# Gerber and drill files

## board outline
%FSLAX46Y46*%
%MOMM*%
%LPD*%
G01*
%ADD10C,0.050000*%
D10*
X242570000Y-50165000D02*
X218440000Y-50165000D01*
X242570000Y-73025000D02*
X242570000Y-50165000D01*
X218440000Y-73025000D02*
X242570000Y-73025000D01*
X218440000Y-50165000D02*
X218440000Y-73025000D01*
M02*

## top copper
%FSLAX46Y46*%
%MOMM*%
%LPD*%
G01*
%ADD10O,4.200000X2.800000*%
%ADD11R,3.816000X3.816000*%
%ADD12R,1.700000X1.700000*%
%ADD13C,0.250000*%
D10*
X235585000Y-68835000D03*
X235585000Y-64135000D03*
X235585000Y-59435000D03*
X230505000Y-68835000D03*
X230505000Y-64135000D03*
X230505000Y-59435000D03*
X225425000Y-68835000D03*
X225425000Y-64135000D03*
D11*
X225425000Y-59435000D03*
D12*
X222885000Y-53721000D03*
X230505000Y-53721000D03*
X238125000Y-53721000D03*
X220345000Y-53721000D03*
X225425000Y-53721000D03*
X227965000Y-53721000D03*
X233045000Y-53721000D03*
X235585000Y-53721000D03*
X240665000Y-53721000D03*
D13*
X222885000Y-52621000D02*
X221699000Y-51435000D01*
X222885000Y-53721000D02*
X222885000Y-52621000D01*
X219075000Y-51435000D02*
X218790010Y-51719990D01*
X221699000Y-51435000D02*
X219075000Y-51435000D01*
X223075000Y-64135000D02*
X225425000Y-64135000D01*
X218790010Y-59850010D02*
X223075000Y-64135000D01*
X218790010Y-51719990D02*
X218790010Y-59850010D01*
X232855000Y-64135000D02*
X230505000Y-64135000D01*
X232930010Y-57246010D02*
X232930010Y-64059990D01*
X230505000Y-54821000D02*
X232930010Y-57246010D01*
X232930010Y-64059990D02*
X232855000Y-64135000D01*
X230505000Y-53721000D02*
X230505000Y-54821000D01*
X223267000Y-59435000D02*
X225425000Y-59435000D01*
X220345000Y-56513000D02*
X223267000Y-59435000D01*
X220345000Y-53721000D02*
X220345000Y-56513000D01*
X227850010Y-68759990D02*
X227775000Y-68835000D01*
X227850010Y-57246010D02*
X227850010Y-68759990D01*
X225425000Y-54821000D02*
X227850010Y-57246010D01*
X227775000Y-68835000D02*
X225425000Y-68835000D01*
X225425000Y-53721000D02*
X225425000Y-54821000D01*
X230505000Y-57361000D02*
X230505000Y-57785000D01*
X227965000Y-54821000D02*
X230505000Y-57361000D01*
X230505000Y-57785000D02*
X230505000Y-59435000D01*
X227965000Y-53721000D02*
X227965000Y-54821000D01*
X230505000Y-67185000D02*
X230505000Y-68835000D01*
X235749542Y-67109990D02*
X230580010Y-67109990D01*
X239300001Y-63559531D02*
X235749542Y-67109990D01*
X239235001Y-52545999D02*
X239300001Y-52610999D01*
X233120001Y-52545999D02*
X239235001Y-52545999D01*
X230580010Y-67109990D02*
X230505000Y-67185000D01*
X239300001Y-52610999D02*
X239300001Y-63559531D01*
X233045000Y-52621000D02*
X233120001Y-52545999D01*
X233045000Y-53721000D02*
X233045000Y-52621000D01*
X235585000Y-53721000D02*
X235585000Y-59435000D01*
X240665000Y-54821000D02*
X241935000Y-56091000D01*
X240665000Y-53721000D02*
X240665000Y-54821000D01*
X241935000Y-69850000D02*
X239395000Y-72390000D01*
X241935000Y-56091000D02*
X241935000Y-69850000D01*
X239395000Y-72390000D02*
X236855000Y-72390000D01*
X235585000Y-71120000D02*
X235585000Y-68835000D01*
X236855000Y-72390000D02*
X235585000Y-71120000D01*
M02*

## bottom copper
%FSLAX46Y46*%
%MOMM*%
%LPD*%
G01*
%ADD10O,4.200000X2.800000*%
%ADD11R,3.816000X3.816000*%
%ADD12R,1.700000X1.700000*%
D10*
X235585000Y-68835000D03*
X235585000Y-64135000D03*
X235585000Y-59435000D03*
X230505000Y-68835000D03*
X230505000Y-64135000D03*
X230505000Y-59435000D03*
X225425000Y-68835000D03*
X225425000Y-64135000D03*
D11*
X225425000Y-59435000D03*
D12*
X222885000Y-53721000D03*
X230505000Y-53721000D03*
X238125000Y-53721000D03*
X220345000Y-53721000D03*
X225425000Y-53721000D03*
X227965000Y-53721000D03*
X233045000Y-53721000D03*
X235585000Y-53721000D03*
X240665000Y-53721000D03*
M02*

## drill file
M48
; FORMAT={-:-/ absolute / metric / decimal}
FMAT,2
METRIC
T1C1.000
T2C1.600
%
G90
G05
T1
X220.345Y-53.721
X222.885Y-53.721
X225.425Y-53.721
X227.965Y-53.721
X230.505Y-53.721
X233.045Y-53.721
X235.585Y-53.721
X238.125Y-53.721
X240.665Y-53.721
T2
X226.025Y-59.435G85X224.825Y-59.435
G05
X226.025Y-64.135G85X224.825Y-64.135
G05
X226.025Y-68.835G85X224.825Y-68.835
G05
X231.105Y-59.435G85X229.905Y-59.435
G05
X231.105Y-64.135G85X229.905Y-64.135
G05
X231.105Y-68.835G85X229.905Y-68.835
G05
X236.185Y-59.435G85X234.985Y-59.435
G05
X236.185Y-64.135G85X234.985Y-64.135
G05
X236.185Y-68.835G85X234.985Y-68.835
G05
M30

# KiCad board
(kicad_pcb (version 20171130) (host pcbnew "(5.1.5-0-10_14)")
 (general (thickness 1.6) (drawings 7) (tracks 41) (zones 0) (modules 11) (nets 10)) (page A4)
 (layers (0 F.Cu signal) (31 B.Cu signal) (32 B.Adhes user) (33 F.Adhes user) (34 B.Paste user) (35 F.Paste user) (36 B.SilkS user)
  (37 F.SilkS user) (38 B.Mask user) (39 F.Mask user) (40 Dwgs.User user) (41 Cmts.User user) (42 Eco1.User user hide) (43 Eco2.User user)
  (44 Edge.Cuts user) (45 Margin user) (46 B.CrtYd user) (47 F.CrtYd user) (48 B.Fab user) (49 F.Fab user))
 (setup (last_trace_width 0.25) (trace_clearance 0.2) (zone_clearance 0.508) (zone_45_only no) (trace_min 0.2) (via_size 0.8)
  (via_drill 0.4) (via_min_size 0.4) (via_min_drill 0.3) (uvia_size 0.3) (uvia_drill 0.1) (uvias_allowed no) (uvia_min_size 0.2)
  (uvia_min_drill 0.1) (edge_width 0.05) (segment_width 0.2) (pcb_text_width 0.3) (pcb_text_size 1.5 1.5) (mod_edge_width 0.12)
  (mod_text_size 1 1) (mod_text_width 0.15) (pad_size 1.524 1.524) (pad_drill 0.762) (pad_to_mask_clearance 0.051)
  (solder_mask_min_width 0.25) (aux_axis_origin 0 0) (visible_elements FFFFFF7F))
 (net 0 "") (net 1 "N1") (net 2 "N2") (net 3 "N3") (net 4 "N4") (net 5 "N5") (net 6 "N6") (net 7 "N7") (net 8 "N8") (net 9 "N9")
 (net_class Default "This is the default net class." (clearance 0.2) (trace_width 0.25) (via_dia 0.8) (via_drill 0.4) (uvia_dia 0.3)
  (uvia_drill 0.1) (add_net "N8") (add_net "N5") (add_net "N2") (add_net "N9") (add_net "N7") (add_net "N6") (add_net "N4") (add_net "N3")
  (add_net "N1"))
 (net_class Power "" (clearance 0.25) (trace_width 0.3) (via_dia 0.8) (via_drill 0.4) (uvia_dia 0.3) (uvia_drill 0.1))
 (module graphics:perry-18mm (layer F.Cu) (at 229.87 62.865)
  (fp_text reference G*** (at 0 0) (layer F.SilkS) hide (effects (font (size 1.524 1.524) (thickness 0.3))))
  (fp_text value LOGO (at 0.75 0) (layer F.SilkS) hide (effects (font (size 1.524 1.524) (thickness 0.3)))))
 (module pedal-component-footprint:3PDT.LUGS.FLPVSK (layer F.Cu) (at 230.505 64.135)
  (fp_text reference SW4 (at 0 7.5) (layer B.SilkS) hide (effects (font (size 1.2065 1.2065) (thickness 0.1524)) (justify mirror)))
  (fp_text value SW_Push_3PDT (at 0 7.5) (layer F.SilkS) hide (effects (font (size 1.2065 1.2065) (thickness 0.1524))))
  (pad 9 thru_hole oval (at 5.08 4.7 180) (size 4.2 2.8) (drill oval 2.8 1.6) (layers *.Cu *.Mask) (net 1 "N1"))
  (pad 8 thru_hole oval (at 5.08 0 180) (size 4.2 2.8) (drill oval 2.8 1.6) (layers *.Cu *.Mask) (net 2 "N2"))
  (pad 7 thru_hole oval (at 5.08 -4.7 180) (size 4.2 2.8) (drill oval 2.8 1.6) (layers *.Cu *.Mask) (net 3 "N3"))
  (pad 6 thru_hole oval (at 0 4.7 180) (size 4.2 2.8) (drill oval 2.8 1.6) (layers *.Cu *.Mask) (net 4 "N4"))
  (pad 5 thru_hole oval (at 0 0 180) (size 4.2 2.8) (drill oval 2.8 1.6) (layers *.Cu *.Mask) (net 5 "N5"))
  (pad 4 thru_hole oval (at 0 -4.7 180) (size 4.2 2.8) (drill oval 2.8 1.6) (layers *.Cu *.Mask) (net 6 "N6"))
  (pad 3 thru_hole oval (at -5.08 4.7 180) (size 4.2 2.8) (drill oval 2.8 1.6) (layers *.Cu *.Mask) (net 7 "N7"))
  (pad 2 thru_hole oval (at -5.08 0 180) (size 4.2 2.8) (drill oval 2.8 1.6) (layers *.Cu *.Mask) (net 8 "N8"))
  (pad 1 thru_hole rect (at -5.08 -4.7 180) (size 3.816 3.816) (drill oval 2.8 1.6) (layers *.Cu *.Mask) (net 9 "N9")))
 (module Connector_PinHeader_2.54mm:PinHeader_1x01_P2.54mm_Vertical (layer F.Cu) (at 222.885 53.721)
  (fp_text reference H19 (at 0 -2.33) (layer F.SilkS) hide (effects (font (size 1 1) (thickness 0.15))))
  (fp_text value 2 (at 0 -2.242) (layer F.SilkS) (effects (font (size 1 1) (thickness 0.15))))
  (pad 1 thru_hole rect (at 0 0) (size 1.7 1.7) (drill 1) (layers *.Cu *.Mask) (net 8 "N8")))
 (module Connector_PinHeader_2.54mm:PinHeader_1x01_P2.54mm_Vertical (layer F.Cu) (at 230.505 53.721)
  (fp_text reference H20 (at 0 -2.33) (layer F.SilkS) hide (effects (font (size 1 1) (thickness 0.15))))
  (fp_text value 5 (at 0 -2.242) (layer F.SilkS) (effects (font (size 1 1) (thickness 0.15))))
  (pad 1 thru_hole rect (at 0 0) (size 1.7 1.7) (drill 1) (layers *.Cu *.Mask) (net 5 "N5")))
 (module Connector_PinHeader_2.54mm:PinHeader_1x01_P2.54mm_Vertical (layer F.Cu) (at 238.125 53.721)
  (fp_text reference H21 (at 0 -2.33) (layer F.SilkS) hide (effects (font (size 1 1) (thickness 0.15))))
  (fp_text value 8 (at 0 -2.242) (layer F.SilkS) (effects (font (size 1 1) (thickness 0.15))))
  (pad 1 thru_hole rect (at 0 0) (size 1.7 1.7) (drill 1) (layers *.Cu *.Mask) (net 2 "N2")))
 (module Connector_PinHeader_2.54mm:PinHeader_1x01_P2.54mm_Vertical (layer F.Cu) (at 220.345 53.721)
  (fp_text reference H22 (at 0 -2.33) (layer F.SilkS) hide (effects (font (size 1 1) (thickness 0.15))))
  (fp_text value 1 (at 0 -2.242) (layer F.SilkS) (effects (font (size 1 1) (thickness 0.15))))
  (pad 1 thru_hole rect (at 0 0) (size 1.7 1.7) (drill 1) (layers *.Cu *.Mask) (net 9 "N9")))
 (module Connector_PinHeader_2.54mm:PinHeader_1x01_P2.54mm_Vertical (layer F.Cu) (at 225.425 53.721)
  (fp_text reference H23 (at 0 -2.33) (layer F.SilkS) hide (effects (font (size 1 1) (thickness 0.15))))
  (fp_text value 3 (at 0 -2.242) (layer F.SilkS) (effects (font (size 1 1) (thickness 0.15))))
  (pad 1 thru_hole rect (at 0 0) (size 1.7 1.7) (drill 1) (layers *.Cu *.Mask) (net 7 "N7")))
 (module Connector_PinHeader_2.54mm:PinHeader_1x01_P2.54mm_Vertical (layer F.Cu) (at 227.965 53.721)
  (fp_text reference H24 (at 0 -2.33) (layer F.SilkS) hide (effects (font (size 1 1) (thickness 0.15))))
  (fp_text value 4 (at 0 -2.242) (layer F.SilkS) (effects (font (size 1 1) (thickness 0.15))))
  (pad 1 thru_hole rect (at 0 0) (size 1.7 1.7) (drill 1) (layers *.Cu *.Mask) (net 6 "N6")))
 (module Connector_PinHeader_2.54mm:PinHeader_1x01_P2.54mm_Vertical (layer F.Cu) (at 233.045 53.721)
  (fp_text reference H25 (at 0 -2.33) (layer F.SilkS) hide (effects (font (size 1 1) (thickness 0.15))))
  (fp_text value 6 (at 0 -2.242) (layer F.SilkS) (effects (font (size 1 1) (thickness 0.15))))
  (pad 1 thru_hole rect (at 0 0) (size 1.7 1.7) (drill 1) (layers *.Cu *.Mask) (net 4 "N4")))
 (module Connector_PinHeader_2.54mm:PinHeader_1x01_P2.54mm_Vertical (layer F.Cu) (at 235.585 53.721)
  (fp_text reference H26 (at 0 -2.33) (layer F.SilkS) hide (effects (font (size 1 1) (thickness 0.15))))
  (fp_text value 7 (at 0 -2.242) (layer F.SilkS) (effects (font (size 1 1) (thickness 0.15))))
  (pad 1 thru_hole rect (at 0 0) (size 1.7 1.7) (drill 1) (layers *.Cu *.Mask) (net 3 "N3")))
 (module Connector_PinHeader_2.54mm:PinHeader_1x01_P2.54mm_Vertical (layer F.Cu) (at 240.665 53.721)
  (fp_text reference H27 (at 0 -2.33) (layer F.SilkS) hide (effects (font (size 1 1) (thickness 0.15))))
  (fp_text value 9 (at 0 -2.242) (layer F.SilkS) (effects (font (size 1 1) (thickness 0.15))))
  (pad 1 thru_hole rect (at 0 0) (size 1.7 1.7) (drill 1) (layers *.Cu *.Mask) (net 1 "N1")))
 (gr_line (start 242.57 50.165) (end 218.44 50.165) (layer Edge.Cuts) (width 0.05))
 (gr_line (start 242.57 73.025) (end 242.57 50.165) (layer Edge.Cuts) (width 0.05))
 (gr_line (start 218.44 73.025) (end 242.57 73.025) (layer Edge.Cuts) (width 0.05))
 (gr_line (start 218.44 50.165) (end 218.44 73.025) (layer Edge.Cuts) (width 0.05))
 (segment (start 222.885 52.621) (end 221.699 51.435) (width 0.25) (layer F.Cu) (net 8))
 (segment (start 222.885 53.721) (end 222.885 52.621) (width 0.25) (layer F.Cu) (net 8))
 (segment (start 219.075 51.435) (end 218.79001 51.71999) (width 0.25) (layer F.Cu) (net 8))
 (segment (start 221.699 51.435) (end 219.075 51.435) (width 0.25) (layer F.Cu) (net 8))
 (segment (start 223.075 64.135) (end 225.425 64.135) (width 0.25) (layer F.Cu) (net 8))
 (segment (start 218.79001 59.85001) (end 223.075 64.135) (width 0.25) (layer F.Cu) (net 8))
 (segment (start 218.79001 51.71999) (end 218.79001 59.85001) (width 0.25) (layer F.Cu) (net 8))
 (segment (start 232.855 64.135) (end 230.505 64.135) (width 0.25) (layer F.Cu) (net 5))
 (segment (start 232.93001 57.24601) (end 232.93001 64.05999) (width 0.25) (layer F.Cu) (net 5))
 (segment (start 230.505 54.821) (end 232.93001 57.24601) (width 0.25) (layer F.Cu) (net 5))
 (segment (start 232.93001 64.05999) (end 232.855 64.135) (width 0.25) (layer F.Cu) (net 5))
 (segment (start 230.505 53.721) (end 230.505 54.821) (width 0.25) (layer F.Cu) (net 5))
 (segment (start 223.267 59.435) (end 225.425 59.435) (width 0.25) (layer F.Cu) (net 9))
 (segment (start 220.345 56.513) (end 223.267 59.435) (width 0.25) (layer F.Cu) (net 9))
 (segment (start 220.345 53.721) (end 220.345 56.513) (width 0.25) (layer F.Cu) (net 9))
 (segment (start 227.85001 68.75999) (end 227.775 68.835) (width 0.25) (layer F.Cu) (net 7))
 (segment (start 227.85001 57.24601) (end 227.85001 68.75999) (width 0.25) (layer F.Cu) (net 7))
 (segment (start 225.425 54.821) (end 227.85001 57.24601) (width 0.25) (layer F.Cu) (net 7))
 (segment (start 227.775 68.835) (end 225.425 68.835) (width 0.25) (layer F.Cu) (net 7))
 (segment (start 225.425 53.721) (end 225.425 54.821) (width 0.25) (layer F.Cu) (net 7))
 (segment (start 230.505 57.361) (end 230.505 57.785) (width 0.25) (layer F.Cu) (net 6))
 (segment (start 227.965 54.821) (end 230.505 57.361) (width 0.25) (layer F.Cu) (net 6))
 (segment (start 230.505 57.785) (end 230.505 59.435) (width 0.25) (layer F.Cu) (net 6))
 (segment (start 227.965 53.721) (end 227.965 54.821) (width 0.25) (layer F.Cu) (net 6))
 (segment (start 230.505 67.185) (end 230.505 68.835) (width 0.25) (layer F.Cu) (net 4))
 (segment (start 235.749542 67.10999) (end 230.58001 67.10999) (width 0.25) (layer F.Cu) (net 4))
 (segment (start 239.300001 63.559531) (end 235.749542 67.10999) (width 0.25) (layer F.Cu) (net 4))
 (segment (start 239.235001 52.545999) (end 239.300001 52.610999) (width 0.25) (layer F.Cu) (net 4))
 (segment (start 233.120001 52.545999) (end 239.235001 52.545999) (width 0.25) (layer F.Cu) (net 4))
 (segment (start 230.58001 67.10999) (end 230.505 67.185) (width 0.25) (layer F.Cu) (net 4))
 (segment (start 239.300001 52.610999) (end 239.300001 63.559531) (width 0.25) (layer F.Cu) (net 4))
 (segment (start 233.045 52.621) (end 233.120001 52.545999) (width 0.25) (layer F.Cu) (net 4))
 (segment (start 233.045 53.721) (end 233.045 52.621) (width 0.25) (layer F.Cu) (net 4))
 (segment (start 235.585 53.721) (end 235.585 59.435) (width 0.25) (layer F.Cu) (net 3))
 (segment (start 240.665 54.821) (end 241.935 56.091) (width 0.25) (layer F.Cu) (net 1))
 (segment (start 240.665 53.721) (end 240.665 54.821) (width 0.25) (layer F.Cu) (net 1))
 (segment (start 241.935 69.85) (end 239.395 72.39) (width 0.25) (layer F.Cu) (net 1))
 (segment (start 241.935 56.091) (end 241.935 69.85) (width 0.25) (layer F.Cu) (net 1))
 (segment (start 239.395 72.39) (end 236.855 72.39) (width 0.25) (layer F.Cu) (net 1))
 (segment (start 235.585 71.12) (end 235.585 68.835) (width 0.25) (layer F.Cu) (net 1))
 (segment (start 236.855 72.39) (end 235.585 71.12) (width 0.25) (layer F.Cu) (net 1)))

